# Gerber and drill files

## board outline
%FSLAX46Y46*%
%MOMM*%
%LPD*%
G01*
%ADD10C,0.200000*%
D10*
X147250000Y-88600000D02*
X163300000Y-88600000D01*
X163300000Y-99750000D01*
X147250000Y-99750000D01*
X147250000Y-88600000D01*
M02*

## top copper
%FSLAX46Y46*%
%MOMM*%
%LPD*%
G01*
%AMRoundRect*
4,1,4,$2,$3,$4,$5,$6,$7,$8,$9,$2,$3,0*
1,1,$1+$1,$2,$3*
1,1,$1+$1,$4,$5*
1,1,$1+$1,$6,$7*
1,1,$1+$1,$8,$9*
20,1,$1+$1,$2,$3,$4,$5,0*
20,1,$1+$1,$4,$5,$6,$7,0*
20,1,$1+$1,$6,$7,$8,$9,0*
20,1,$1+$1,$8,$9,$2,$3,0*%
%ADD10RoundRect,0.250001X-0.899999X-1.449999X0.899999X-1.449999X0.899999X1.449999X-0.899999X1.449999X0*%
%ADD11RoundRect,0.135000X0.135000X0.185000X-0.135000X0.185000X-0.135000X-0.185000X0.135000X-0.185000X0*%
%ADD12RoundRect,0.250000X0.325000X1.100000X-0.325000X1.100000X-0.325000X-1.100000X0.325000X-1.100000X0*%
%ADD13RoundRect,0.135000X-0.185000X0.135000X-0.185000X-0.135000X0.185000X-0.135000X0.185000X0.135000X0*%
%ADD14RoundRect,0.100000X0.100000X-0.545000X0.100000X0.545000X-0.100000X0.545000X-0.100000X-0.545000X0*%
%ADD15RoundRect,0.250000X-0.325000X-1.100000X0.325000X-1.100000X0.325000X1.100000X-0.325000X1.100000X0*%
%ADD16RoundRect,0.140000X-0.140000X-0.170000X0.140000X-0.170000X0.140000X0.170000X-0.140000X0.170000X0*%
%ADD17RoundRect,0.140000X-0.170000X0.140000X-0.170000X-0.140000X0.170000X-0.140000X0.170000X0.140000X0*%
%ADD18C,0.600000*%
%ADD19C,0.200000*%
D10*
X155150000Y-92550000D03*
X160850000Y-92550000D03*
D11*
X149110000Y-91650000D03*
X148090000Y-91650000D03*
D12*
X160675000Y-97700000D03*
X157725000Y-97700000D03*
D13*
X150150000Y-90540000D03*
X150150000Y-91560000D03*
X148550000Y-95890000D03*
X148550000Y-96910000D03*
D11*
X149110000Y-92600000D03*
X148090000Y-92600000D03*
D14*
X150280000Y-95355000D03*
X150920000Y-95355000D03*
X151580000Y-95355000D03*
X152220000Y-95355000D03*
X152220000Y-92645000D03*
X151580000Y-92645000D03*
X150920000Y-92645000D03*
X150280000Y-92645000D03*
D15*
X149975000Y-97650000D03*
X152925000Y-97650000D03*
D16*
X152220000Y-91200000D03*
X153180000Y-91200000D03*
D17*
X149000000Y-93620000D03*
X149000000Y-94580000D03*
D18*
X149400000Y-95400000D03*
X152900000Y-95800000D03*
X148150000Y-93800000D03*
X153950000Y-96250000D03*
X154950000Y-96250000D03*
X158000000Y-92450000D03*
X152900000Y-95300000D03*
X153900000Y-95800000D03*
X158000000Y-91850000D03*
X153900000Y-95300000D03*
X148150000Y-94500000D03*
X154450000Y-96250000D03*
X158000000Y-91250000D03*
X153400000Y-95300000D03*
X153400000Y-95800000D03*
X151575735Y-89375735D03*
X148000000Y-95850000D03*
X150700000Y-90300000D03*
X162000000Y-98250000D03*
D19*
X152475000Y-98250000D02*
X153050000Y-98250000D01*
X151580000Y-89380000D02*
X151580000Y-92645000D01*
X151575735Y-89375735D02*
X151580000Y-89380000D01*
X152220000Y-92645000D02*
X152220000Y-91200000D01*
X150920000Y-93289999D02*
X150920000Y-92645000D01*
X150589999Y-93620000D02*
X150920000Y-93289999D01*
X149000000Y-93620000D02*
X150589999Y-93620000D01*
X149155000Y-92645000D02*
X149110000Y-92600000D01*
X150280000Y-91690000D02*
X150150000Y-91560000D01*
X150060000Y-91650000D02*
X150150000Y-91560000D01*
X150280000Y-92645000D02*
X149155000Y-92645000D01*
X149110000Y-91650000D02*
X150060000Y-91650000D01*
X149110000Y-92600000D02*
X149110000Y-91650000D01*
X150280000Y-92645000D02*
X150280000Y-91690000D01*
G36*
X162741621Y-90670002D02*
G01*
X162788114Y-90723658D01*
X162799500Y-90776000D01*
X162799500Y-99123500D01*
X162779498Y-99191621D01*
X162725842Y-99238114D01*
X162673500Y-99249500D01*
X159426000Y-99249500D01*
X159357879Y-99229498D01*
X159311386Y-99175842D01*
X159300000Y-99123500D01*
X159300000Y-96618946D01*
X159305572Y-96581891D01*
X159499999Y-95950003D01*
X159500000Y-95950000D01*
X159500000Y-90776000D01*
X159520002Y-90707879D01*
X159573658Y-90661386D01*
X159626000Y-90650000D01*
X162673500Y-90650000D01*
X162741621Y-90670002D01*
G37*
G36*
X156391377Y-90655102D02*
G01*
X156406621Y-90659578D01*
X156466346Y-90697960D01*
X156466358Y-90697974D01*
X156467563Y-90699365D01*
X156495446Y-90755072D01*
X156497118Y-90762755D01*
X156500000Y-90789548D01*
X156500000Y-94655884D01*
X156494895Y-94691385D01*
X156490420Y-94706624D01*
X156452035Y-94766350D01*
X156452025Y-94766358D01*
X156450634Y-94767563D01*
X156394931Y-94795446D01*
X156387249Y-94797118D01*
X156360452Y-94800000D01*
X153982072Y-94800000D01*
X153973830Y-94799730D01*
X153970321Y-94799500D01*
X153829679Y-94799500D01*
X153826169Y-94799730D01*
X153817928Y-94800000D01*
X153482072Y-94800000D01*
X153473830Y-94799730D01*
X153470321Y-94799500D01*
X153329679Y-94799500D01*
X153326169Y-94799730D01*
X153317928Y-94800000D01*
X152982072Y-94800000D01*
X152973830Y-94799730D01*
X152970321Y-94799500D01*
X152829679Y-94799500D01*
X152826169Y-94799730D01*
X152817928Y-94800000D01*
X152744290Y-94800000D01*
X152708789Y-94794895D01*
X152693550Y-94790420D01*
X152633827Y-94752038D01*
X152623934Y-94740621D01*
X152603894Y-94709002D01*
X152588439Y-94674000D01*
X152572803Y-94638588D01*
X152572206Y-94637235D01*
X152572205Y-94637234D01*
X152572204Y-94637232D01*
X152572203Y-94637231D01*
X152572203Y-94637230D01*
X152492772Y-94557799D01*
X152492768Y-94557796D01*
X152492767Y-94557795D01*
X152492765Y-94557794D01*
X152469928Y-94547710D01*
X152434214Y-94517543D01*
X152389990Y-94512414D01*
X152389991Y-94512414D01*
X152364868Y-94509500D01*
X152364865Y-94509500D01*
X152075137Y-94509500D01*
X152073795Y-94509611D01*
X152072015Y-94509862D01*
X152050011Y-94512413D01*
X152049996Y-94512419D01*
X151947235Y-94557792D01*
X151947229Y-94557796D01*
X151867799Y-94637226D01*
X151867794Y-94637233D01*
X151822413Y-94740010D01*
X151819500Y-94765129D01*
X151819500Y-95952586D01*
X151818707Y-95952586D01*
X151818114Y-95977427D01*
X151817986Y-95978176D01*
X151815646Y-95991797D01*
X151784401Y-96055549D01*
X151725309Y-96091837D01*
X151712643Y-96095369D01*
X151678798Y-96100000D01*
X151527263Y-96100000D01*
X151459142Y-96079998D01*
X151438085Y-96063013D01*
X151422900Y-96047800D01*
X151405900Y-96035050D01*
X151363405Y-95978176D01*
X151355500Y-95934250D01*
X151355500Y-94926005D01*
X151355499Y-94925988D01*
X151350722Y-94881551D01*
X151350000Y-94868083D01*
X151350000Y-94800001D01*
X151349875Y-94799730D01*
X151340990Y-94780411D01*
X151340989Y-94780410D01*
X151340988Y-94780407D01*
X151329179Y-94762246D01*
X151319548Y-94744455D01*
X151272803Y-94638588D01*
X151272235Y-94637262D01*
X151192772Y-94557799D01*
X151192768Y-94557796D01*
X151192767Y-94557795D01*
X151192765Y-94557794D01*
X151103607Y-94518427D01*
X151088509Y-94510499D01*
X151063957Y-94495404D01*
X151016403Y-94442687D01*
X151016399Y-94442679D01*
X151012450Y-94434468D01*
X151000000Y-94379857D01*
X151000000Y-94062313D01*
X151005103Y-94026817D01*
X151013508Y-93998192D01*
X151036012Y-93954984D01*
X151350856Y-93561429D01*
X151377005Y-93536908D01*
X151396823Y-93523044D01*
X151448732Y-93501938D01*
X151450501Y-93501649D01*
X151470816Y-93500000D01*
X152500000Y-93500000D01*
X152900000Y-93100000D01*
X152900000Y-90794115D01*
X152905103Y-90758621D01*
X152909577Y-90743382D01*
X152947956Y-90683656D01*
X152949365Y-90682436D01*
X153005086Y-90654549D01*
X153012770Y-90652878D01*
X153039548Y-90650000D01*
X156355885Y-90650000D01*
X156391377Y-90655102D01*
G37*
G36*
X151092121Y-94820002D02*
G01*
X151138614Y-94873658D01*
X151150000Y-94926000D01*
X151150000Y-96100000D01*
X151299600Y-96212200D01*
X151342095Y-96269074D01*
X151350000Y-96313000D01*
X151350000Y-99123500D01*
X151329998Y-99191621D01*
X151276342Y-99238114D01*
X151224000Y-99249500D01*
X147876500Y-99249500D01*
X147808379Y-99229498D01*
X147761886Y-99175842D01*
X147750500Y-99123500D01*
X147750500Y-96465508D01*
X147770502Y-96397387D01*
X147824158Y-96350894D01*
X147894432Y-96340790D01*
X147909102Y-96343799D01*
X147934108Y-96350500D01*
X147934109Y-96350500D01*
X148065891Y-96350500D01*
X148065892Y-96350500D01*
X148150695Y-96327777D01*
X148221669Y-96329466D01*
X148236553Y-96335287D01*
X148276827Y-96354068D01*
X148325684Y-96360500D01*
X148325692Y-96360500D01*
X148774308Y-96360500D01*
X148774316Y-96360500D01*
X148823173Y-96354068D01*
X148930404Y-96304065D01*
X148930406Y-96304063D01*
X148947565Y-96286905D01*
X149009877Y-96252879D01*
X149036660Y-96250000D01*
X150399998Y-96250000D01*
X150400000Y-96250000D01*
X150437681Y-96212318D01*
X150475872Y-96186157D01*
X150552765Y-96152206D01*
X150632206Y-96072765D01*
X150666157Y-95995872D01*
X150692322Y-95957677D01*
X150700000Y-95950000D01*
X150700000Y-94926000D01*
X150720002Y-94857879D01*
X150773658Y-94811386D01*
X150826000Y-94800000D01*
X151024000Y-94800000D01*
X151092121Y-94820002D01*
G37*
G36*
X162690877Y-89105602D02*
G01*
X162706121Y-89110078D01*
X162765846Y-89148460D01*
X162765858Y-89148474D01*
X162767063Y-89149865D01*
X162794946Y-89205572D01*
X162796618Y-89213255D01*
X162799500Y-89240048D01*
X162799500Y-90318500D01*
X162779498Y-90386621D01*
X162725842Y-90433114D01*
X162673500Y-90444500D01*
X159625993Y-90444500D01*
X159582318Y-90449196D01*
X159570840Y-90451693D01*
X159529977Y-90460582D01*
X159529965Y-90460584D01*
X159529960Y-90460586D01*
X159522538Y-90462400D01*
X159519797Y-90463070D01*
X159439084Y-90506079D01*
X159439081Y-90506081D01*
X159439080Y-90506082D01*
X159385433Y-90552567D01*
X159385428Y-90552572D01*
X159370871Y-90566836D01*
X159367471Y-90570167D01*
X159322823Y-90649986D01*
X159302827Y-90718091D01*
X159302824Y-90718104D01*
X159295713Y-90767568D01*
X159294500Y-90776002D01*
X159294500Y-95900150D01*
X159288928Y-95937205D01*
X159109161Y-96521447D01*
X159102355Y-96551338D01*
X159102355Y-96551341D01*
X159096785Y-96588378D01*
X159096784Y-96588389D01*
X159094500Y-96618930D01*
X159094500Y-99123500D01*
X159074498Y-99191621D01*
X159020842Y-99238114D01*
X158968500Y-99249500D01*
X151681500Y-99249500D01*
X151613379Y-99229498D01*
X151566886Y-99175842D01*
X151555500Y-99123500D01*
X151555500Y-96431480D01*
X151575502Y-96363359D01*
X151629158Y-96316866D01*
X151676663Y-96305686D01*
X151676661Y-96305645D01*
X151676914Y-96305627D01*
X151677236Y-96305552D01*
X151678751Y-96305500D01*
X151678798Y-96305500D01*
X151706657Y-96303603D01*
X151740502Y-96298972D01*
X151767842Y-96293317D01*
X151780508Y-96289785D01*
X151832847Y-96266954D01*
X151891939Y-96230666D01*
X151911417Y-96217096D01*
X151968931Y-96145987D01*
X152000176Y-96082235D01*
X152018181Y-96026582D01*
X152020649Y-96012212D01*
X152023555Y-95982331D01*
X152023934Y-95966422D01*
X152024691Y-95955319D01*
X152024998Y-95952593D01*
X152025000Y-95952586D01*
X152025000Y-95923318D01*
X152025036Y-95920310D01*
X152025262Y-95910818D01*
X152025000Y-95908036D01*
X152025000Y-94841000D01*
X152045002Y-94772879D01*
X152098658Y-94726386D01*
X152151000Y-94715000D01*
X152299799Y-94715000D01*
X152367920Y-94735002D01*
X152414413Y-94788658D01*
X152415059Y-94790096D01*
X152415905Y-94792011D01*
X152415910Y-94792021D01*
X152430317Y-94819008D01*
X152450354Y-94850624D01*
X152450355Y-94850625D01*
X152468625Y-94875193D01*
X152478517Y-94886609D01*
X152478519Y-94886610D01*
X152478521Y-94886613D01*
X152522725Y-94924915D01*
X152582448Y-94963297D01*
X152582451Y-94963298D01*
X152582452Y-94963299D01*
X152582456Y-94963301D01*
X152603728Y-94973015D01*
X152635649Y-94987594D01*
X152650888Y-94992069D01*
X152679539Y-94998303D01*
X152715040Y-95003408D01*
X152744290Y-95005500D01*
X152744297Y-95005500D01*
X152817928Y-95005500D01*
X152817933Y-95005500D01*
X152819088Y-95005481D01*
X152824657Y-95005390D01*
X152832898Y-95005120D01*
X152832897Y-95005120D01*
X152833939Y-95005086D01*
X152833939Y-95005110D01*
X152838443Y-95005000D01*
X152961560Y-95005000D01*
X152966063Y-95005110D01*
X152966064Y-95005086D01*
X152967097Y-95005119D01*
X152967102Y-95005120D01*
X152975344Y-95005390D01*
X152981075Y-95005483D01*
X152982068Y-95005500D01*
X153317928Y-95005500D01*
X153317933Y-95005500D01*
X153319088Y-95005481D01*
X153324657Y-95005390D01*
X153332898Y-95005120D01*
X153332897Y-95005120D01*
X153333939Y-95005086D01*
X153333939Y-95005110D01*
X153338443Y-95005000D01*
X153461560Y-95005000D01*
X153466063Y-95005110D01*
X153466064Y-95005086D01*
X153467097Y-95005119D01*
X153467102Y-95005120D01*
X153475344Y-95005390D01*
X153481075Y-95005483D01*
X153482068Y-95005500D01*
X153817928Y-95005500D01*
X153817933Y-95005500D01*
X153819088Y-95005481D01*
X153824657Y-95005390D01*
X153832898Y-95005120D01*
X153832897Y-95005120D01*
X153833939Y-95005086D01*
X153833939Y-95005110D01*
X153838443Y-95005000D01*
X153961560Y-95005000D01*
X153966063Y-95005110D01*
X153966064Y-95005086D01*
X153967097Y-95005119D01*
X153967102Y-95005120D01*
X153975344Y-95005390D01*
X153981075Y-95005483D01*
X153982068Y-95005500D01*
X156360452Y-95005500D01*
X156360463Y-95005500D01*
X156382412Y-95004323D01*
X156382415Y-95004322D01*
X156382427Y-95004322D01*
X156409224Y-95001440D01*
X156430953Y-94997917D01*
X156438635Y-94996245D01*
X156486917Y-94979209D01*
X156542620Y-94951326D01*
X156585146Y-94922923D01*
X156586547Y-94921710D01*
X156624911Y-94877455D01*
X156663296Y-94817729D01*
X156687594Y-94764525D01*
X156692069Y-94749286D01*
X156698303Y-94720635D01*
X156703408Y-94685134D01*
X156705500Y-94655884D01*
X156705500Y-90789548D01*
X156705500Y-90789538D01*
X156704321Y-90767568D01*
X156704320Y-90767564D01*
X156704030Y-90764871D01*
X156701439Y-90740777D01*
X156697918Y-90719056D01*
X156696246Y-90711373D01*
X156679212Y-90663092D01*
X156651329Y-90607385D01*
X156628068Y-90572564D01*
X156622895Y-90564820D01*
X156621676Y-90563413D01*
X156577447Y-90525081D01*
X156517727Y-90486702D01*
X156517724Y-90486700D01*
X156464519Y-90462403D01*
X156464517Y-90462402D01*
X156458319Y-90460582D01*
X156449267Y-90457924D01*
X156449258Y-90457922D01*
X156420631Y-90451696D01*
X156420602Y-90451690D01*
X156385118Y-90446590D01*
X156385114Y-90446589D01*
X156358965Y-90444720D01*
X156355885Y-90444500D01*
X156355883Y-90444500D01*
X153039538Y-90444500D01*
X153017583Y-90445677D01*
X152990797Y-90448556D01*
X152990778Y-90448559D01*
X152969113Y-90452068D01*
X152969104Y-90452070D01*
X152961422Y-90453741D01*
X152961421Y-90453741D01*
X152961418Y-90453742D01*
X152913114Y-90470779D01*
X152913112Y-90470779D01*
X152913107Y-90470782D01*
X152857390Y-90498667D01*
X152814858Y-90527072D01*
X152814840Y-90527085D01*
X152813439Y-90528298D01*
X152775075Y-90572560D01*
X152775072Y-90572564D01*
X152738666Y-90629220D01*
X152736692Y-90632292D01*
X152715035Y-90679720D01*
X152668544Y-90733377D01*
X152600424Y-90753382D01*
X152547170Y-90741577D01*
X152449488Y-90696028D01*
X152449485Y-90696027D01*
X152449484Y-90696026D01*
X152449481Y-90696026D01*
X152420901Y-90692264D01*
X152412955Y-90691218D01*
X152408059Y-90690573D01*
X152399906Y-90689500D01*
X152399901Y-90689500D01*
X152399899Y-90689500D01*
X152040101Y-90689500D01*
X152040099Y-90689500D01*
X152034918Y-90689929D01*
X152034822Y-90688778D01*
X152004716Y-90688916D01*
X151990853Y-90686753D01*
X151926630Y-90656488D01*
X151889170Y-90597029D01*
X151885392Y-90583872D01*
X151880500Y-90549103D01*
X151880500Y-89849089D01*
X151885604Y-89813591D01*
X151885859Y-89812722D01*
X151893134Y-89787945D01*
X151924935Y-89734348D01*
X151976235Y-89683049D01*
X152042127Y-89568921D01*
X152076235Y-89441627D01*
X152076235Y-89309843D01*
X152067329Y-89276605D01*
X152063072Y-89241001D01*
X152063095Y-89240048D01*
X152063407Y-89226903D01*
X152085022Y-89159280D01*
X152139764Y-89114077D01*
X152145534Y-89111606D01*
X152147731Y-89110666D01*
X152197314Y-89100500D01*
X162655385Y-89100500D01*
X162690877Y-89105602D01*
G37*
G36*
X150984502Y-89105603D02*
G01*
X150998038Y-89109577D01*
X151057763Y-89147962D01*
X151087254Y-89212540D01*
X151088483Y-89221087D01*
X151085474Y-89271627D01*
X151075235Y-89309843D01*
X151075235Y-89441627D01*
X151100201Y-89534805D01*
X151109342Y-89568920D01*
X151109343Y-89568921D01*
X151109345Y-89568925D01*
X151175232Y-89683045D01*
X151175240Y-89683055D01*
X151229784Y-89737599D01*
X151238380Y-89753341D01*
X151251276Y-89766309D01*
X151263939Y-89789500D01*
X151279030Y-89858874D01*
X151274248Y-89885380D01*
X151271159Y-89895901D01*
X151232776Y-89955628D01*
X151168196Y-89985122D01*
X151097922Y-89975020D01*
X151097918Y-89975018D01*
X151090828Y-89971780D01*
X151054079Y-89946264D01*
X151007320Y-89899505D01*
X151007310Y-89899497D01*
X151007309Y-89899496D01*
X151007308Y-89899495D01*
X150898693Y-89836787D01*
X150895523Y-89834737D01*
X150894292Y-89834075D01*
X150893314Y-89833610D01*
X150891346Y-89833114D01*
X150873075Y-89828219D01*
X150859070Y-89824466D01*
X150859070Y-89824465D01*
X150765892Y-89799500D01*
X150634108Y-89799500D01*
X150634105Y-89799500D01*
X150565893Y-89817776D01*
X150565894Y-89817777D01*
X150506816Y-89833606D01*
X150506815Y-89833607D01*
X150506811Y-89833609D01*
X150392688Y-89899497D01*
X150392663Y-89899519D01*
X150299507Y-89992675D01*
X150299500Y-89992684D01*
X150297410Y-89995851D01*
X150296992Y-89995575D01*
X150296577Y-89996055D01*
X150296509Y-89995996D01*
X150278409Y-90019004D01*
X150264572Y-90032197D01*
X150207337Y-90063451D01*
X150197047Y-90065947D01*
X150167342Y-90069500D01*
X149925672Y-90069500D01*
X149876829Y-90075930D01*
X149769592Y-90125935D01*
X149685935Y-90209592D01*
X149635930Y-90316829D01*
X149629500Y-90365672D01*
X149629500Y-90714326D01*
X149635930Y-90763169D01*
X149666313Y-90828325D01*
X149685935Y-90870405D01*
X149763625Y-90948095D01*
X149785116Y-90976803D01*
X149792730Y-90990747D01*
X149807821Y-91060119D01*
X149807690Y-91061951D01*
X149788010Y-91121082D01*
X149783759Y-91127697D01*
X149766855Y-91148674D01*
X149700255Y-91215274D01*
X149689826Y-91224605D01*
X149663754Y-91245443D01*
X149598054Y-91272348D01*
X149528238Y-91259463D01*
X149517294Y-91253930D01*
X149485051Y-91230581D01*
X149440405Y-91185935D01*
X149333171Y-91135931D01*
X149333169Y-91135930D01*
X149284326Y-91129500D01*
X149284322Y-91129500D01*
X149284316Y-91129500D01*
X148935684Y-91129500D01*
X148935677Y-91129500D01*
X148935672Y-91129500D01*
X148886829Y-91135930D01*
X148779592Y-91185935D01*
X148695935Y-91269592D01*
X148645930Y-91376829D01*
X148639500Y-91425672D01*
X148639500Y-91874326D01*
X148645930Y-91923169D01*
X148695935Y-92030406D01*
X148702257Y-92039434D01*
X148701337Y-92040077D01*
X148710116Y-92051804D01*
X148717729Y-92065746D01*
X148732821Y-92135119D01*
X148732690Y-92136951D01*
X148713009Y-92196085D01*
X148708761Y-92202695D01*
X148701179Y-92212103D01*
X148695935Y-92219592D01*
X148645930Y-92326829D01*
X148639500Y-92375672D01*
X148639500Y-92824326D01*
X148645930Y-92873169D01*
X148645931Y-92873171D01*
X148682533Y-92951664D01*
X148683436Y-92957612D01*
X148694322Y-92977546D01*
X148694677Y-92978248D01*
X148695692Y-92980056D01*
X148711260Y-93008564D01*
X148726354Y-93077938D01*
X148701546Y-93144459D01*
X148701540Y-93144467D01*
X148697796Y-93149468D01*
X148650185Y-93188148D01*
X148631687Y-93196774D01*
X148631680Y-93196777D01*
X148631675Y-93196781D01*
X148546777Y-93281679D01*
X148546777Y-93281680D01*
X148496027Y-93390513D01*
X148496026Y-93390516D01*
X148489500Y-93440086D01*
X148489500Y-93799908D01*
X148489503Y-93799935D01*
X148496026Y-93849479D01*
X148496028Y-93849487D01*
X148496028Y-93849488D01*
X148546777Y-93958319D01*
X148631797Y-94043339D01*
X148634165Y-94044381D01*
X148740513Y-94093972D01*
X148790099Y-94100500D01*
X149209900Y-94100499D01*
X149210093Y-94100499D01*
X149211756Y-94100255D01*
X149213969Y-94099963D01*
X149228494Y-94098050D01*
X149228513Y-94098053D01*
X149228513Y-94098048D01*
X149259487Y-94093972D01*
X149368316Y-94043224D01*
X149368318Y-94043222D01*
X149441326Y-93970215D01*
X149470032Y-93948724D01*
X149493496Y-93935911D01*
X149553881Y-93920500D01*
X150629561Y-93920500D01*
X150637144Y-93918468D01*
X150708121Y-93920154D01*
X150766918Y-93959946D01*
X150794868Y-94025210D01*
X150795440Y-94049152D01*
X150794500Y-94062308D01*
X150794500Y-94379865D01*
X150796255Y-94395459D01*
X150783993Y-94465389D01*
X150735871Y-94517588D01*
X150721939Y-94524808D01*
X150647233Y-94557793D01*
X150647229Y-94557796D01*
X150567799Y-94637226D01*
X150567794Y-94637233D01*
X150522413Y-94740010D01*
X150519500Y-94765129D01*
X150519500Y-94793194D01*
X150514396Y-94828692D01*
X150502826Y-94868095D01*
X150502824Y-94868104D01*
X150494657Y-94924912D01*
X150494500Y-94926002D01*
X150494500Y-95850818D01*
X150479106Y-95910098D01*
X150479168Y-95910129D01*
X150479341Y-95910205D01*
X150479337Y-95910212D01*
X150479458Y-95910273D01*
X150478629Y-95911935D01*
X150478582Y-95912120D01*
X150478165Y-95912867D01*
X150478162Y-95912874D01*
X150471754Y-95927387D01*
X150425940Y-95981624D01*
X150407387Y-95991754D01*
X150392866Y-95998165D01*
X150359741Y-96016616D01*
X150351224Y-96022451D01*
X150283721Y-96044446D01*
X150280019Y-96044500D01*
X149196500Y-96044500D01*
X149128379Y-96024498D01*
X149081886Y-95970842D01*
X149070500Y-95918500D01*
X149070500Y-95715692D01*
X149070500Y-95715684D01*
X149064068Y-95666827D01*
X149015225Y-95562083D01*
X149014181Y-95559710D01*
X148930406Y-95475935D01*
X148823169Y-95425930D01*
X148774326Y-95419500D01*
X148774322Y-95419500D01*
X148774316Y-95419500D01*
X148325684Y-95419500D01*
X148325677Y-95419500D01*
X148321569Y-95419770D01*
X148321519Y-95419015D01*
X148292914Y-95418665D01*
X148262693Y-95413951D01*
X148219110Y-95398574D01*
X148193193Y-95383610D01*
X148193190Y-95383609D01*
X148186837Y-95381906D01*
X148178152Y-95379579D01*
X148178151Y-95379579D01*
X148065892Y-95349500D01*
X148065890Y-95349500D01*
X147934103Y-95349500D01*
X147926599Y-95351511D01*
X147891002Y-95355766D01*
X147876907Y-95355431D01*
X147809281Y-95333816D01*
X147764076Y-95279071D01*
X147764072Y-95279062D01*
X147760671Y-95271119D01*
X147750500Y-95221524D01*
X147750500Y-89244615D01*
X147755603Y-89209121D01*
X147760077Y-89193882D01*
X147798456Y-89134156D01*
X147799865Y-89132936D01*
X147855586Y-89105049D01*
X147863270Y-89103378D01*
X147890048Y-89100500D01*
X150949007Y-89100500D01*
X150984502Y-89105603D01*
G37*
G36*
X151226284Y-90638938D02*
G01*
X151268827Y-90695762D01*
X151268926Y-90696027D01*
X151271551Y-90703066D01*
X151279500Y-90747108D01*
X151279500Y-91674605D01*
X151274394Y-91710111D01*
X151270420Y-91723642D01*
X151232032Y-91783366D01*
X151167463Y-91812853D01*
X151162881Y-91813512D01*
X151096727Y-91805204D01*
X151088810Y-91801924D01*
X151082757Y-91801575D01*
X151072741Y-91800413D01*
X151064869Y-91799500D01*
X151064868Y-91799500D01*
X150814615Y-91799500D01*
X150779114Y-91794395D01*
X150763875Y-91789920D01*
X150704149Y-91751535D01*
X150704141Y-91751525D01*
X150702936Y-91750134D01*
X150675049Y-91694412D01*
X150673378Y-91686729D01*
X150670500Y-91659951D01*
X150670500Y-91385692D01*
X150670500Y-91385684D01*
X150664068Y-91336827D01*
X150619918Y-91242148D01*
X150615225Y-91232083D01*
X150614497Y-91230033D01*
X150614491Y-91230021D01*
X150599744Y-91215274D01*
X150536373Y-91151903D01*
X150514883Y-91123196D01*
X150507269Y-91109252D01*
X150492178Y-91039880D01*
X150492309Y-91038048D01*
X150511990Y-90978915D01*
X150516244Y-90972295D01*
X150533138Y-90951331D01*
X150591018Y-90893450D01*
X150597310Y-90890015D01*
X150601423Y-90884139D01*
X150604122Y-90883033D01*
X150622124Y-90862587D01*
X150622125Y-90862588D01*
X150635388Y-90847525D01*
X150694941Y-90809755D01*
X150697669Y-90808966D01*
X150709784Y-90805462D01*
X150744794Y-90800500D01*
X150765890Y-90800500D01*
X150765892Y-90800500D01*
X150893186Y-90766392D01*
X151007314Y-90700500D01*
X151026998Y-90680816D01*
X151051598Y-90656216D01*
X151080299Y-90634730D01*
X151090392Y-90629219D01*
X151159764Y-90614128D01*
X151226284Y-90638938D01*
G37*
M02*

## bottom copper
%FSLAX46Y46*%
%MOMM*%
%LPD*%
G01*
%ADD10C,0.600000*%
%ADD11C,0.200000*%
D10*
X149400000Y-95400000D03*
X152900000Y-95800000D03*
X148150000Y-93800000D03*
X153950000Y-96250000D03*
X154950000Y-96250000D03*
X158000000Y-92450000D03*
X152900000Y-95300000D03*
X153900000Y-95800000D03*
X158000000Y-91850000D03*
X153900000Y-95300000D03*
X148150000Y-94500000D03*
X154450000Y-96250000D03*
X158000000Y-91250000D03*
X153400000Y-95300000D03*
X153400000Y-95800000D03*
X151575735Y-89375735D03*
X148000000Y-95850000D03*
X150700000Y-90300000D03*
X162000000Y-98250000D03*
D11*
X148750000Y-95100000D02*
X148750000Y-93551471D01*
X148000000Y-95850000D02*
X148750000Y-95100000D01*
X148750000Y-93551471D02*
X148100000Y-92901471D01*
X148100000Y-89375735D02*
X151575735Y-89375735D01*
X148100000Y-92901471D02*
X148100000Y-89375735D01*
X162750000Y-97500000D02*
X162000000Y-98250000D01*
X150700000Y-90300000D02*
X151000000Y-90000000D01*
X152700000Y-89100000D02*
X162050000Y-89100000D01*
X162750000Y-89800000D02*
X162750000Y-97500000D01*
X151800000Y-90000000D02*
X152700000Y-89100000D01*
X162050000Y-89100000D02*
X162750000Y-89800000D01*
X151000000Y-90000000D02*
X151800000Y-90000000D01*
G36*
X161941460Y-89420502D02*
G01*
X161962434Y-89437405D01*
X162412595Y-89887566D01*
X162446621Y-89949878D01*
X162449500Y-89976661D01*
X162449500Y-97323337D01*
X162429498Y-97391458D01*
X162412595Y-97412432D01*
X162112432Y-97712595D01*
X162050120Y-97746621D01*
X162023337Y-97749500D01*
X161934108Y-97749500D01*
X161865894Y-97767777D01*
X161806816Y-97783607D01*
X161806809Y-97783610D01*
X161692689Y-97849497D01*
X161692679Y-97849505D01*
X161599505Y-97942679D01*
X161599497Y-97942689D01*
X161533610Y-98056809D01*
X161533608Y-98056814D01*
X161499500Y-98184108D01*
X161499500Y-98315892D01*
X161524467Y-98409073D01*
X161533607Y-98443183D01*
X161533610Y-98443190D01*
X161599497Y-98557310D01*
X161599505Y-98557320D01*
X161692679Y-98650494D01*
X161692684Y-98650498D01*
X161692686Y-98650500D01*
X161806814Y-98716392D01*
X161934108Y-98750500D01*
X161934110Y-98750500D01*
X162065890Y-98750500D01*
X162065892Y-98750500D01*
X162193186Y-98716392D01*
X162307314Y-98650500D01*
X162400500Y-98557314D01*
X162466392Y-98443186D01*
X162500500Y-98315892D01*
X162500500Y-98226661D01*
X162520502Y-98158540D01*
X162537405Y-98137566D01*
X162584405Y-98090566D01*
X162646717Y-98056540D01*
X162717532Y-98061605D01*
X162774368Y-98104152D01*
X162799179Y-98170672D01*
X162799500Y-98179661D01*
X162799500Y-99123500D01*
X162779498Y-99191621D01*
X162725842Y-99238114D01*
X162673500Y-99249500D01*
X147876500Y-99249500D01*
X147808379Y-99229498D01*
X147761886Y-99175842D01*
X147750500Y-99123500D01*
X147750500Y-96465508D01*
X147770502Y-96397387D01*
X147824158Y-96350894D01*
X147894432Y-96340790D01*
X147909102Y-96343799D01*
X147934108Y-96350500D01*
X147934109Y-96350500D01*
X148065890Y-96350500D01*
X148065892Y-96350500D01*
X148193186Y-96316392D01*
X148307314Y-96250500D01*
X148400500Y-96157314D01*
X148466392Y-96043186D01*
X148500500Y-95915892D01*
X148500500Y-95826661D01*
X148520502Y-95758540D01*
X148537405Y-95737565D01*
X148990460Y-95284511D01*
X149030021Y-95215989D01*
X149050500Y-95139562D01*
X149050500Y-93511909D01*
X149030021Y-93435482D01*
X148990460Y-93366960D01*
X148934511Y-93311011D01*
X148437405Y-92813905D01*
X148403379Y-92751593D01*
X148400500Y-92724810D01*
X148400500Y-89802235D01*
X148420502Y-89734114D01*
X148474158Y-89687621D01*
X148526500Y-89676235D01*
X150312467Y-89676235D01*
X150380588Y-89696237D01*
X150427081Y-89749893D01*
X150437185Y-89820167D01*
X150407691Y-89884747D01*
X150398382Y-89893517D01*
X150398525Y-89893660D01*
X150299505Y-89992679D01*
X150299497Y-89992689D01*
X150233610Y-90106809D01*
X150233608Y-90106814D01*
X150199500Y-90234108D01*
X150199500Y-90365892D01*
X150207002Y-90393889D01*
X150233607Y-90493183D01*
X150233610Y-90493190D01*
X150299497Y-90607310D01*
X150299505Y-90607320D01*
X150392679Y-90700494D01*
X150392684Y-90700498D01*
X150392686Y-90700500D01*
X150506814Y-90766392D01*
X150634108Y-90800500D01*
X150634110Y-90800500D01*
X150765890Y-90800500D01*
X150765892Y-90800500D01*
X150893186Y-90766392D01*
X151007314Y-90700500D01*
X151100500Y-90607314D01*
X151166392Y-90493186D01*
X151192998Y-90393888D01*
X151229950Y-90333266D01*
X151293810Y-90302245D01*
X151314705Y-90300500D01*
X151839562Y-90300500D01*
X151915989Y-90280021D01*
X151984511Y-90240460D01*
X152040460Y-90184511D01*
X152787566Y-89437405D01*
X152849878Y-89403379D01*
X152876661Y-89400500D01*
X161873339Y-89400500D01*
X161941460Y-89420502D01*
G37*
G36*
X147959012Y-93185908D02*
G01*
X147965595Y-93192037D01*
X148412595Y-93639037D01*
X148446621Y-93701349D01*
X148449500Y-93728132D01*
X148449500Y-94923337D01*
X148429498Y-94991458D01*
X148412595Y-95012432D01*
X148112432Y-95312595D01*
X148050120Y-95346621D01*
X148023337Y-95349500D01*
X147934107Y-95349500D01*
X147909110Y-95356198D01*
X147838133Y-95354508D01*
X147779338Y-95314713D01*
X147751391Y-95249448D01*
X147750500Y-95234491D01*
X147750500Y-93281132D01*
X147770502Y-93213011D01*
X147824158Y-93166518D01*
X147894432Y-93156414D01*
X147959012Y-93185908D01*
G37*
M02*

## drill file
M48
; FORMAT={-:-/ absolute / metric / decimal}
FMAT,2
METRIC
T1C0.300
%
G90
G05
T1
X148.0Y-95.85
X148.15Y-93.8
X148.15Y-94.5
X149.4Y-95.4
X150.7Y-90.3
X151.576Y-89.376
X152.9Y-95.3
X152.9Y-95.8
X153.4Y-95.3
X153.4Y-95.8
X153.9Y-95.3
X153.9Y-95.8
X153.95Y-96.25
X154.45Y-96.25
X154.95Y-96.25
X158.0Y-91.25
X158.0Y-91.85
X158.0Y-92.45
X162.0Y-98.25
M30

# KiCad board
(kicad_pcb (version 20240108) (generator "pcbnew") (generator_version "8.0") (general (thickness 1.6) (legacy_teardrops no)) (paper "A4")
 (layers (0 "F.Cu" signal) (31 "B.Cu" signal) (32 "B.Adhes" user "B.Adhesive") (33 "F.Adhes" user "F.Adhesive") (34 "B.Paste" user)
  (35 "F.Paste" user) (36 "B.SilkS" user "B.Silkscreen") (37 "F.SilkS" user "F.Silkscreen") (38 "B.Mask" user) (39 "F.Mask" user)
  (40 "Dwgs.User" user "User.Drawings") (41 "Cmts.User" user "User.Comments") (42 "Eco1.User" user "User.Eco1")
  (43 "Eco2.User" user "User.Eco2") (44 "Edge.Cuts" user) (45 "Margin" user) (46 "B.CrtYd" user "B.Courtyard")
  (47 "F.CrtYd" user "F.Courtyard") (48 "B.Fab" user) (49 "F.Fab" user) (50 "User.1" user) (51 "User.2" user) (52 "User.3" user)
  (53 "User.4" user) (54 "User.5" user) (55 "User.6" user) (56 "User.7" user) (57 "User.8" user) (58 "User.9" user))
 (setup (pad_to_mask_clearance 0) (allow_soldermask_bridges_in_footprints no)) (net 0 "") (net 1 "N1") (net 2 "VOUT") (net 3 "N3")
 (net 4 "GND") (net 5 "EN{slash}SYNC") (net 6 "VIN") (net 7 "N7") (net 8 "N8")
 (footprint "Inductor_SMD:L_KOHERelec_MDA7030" (layer "F.Cu") (at 158 92.55)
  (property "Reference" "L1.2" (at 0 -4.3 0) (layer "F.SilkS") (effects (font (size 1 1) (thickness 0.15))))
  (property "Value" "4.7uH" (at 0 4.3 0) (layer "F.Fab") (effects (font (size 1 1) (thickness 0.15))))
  (pad "1" smd roundrect (at -2.85 0) (size 2.3 3.4) (layers "F.Cu" "F.Paste" "F.Mask") (roundrect_rratio 0.108696) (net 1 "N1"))
  (pad "2" smd roundrect (at 2.85 0) (size 2.3 3.4) (layers "F.Cu" "F.Paste" "F.Mask") (roundrect_rratio 0.108696) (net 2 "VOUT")))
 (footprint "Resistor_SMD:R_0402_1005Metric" (layer "F.Cu") (at 148.6 91.65 180)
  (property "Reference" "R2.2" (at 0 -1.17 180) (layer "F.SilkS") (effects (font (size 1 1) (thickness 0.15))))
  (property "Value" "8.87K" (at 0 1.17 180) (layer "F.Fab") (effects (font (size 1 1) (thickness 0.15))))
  (pad "1" smd roundrect (at -0.51 0 180) (size 0.54 0.64) (layers "F.Cu" "F.Paste" "F.Mask") (roundrect_rratio 0.25) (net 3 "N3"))
  (pad "2" smd roundrect (at 0.51 0 180) (size 0.54 0.64) (layers "F.Cu" "F.Paste" "F.Mask") (roundrect_rratio 0.25) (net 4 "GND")))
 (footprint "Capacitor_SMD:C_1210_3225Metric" (layer "F.Cu") (at 159.2 97.7 180)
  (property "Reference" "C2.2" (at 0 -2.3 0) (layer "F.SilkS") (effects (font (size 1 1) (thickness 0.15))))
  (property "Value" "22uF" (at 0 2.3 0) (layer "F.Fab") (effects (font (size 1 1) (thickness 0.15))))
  (pad "1" smd roundrect (at -1.475 0 180) (size 1.15 2.7) (layers "F.Cu" "F.Paste" "F.Mask") (roundrect_rratio 0.217391) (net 2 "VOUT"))
  (pad "2" smd roundrect (at 1.475 0 180) (size 1.15 2.7) (layers "F.Cu" "F.Paste" "F.Mask") (roundrect_rratio 0.217391) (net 4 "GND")))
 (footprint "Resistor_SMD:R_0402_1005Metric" (layer "F.Cu") (at 150.15 91.05 -90)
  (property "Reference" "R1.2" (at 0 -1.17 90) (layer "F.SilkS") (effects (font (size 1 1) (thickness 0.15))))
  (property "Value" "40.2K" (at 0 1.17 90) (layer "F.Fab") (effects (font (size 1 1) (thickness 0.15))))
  (pad "1" smd roundrect (at -0.51 0 270) (size 0.54 0.64) (layers "F.Cu" "F.Paste" "F.Mask") (roundrect_rratio 0.25) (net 2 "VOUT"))
  (pad "2" smd roundrect (at 0.51 0 270) (size 0.54 0.64) (layers "F.Cu" "F.Paste" "F.Mask") (roundrect_rratio 0.25) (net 3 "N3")))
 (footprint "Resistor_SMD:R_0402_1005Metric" (layer "F.Cu") (at 148.55 96.4 -90)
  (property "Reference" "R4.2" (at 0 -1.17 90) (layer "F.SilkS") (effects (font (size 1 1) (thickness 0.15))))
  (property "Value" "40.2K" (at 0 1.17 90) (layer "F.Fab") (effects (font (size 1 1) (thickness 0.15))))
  (pad "1" smd roundrect (at -0.51 0 270) (size 0.54 0.64) (layers "F.Cu" "F.Paste" "F.Mask") (roundrect_rratio 0.25)
   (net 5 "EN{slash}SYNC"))
  (pad "2" smd roundrect (at 0.51 0 270) (size 0.54 0.64) (layers "F.Cu" "F.Paste" "F.Mask") (roundrect_rratio 0.25) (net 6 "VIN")))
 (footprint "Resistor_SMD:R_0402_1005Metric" (layer "F.Cu") (at 148.6 92.6 180)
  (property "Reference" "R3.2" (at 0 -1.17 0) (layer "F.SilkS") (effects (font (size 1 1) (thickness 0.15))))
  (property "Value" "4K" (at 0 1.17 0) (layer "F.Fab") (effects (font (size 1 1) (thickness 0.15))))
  (pad "1" smd roundrect (at -0.51 0 180) (size 0.54 0.64) (layers "F.Cu" "F.Paste" "F.Mask") (roundrect_rratio 0.25) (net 3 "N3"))
  (pad "2" smd roundrect (at 0.51 0 180) (size 0.54 0.64) (layers "F.Cu" "F.Paste" "F.Mask") (roundrect_rratio 0.25) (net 4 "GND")))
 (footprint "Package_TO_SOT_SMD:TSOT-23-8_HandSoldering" (layer "F.Cu") (at 151.25 94 90)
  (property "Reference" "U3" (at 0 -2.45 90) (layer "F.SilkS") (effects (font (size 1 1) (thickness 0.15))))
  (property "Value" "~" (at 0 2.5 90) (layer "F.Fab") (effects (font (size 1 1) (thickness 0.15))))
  (pad "1" smd roundrect (at -1.355 -0.97 90) (size 1.29 0.4) (layers "F.Cu" "F.Paste" "F.Mask") (roundrect_rratio 0.25) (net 4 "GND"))
  (pad "2" smd roundrect (at -1.355 -0.33 90) (size 1.29 0.4) (layers "F.Cu" "F.Paste" "F.Mask") (roundrect_rratio 0.25) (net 6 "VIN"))
  (pad "3" smd roundrect (at -1.355 0.33 90) (size 1.29 0.4) (layers "F.Cu" "F.Paste" "F.Mask") (roundrect_rratio 0.25) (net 1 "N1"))
  (pad "4" smd roundrect (at -1.355 0.97 90) (size 1.29 0.4) (layers "F.Cu" "F.Paste" "F.Mask") (roundrect_rratio 0.25) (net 4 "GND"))
  (pad "5" smd roundrect (at 1.355 0.97 90) (size 1.29 0.4) (layers "F.Cu" "F.Paste" "F.Mask") (roundrect_rratio 0.25) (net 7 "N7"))
  (pad "6" smd roundrect (at 1.355 0.33 90) (size 1.29 0.4) (layers "F.Cu" "F.Paste" "F.Mask") (roundrect_rratio 0.25)
   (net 5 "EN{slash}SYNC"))
  (pad "7" smd roundrect (at 1.355 -0.33 90) (size 1.29 0.4) (layers "F.Cu" "F.Paste" "F.Mask") (roundrect_rratio 0.25) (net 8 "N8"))
  (pad "8" smd roundrect (at 1.355 -0.97 90) (size 1.29 0.4) (layers "F.Cu" "F.Paste" "F.Mask") (roundrect_rratio 0.25) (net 3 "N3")))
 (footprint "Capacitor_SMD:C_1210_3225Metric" (layer "F.Cu") (at 151.45 97.65)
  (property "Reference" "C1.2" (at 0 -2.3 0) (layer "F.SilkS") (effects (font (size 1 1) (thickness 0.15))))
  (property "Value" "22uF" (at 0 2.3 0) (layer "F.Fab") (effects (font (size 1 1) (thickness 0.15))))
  (pad "1" smd roundrect (at -1.475 0) (size 1.15 2.7) (layers "F.Cu" "F.Paste" "F.Mask") (roundrect_rratio 0.217391) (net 6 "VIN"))
  (pad "2" smd roundrect (at 1.475 0) (size 1.15 2.7) (layers "F.Cu" "F.Paste" "F.Mask") (roundrect_rratio 0.217391) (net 4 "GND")))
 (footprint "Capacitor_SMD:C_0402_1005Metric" (layer "F.Cu") (at 152.7 91.2)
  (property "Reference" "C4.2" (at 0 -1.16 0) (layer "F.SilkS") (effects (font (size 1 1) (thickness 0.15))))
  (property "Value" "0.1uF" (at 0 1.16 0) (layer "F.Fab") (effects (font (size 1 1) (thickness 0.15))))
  (pad "1" smd roundrect (at -0.48 0) (size 0.56 0.62) (layers "F.Cu" "F.Paste" "F.Mask") (roundrect_rratio 0.25) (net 7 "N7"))
  (pad "2" smd roundrect (at 0.48 0) (size 0.56 0.62) (layers "F.Cu" "F.Paste" "F.Mask") (roundrect_rratio 0.25) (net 1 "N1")))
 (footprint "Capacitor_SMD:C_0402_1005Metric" (layer "F.Cu") (at 149 94.1 -90)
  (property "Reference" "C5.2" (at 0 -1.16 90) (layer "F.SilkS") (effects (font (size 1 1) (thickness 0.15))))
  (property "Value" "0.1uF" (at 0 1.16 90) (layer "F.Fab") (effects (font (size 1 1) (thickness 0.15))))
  (pad "1" smd roundrect (at -0.48 0 270) (size 0.56 0.62) (layers "F.Cu" "F.Paste" "F.Mask") (roundrect_rratio 0.25) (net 8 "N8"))
  (pad "2" smd roundrect (at 0.48 0 270) (size 0.56 0.62) (layers "F.Cu" "F.Paste" "F.Mask") (roundrect_rratio 0.25) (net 4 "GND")))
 (gr_rect (start 147.25 88.6) (end 163.3 99.75) (stroke (width 0.2) (type default)) (fill none) (layer "Edge.Cuts"))
 (segment (start 152.475 98.25) (end 153.05 98.25) (width 0.2) (layer "F.Cu") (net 4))
 (via (at 149.4 95.4) (size 0.6) (drill 0.3) (layers "F.Cu" "B.Cu") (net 4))
 (via (at 152.9 95.8) (size 0.6) (drill 0.3) (layers "F.Cu" "B.Cu") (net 4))
 (via (at 148.15 93.8) (size 0.6) (drill 0.3) (layers "F.Cu" "B.Cu") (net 4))
 (via (at 153.95 96.25) (size 0.6) (drill 0.3) (layers "F.Cu" "B.Cu") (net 4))
 (via (at 154.95 96.25) (size 0.6) (drill 0.3) (layers "F.Cu" "B.Cu") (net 4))
 (via (at 158 92.45) (size 0.6) (drill 0.3) (layers "F.Cu" "B.Cu") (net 4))
 (via (at 152.9 95.3) (size 0.6) (drill 0.3) (layers "F.Cu" "B.Cu") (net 4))
 (via (at 153.9 95.8) (size 0.6) (drill 0.3) (layers "F.Cu" "B.Cu") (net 4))
 (via (at 158 91.85) (size 0.6) (drill 0.3) (layers "F.Cu" "B.Cu") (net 4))
 (via (at 153.9 95.3) (size 0.6) (drill 0.3) (layers "F.Cu" "B.Cu") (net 4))
 (via (at 148.15 94.5) (size 0.6) (drill 0.3) (layers "F.Cu" "B.Cu") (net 4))
 (via (at 154.45 96.25) (size 0.6) (drill 0.3) (layers "F.Cu" "B.Cu") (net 4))
 (via (at 158 91.25) (size 0.6) (drill 0.3) (layers "F.Cu" "B.Cu") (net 4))
 (via (at 153.4 95.3) (size 0.6) (drill 0.3) (layers "F.Cu" "B.Cu") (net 4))
 (via (at 153.4 95.8) (size 0.6) (drill 0.3) (layers "F.Cu" "B.Cu") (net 4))
 (segment (start 151.58 89.38) (end 151.58 92.645) (width 0.2) (layer "F.Cu") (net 5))
 (segment (start 151.575735 89.375735) (end 151.58 89.38) (width 0.2) (layer "F.Cu") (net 5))
 (via (at 151.575735 89.375735) (size 0.6) (drill 0.3) (layers "F.Cu" "B.Cu") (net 5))
 (via (at 148 95.85) (size 0.6) (drill 0.3) (layers "F.Cu" "B.Cu") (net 5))
 (segment (start 148.75 95.1) (end 148.75 93.551471) (width 0.2) (layer "B.Cu") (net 5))
 (segment (start 148 95.85) (end 148.75 95.1) (width 0.2) (layer "B.Cu") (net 5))
 (segment (start 148.75 93.551471) (end 148.1 92.901471) (width 0.2) (layer "B.Cu") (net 5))
 (segment (start 148.1 89.375735) (end 151.575735 89.375735) (width 0.2) (layer "B.Cu") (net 5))
 (segment (start 148.1 92.901471) (end 148.1 89.375735) (width 0.2) (layer "B.Cu") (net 5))
 (via (at 150.7 90.3) (size 0.6) (drill 0.3) (layers "F.Cu" "B.Cu") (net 2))
 (via (at 162 98.25) (size 0.6) (drill 0.3) (layers "F.Cu" "B.Cu") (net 2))
 (segment (start 162.75 97.5) (end 162 98.25) (width 0.2) (layer "B.Cu") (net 2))
 (segment (start 150.7 90.3) (end 151 90) (width 0.2) (layer "B.Cu") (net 2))
 (segment (start 152.7 89.1) (end 162.05 89.1) (width 0.2) (layer "B.Cu") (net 2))
 (segment (start 162.75 89.8) (end 162.75 97.5) (width 0.2) (layer "B.Cu") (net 2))
 (segment (start 151.8 90) (end 152.7 89.1) (width 0.2) (layer "B.Cu") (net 2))
 (segment (start 162.05 89.1) (end 162.75 89.8) (width 0.2) (layer "B.Cu") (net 2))
 (segment (start 151 90) (end 151.8 90) (width 0.2) (layer "B.Cu") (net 2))
 (segment (start 152.22 92.645) (end 152.22 91.2) (width 0.2) (layer "F.Cu") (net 7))
 (segment (start 150.92 93.289999) (end 150.92 92.645) (width 0.2) (layer "F.Cu") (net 8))
 (segment (start 150.589999 93.62) (end 150.92 93.289999) (width 0.2) (layer "F.Cu") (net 8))
 (segment (start 149 93.62) (end 150.589999 93.62) (width 0.2) (layer "F.Cu") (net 8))
 (segment (start 149.155 92.645) (end 149.11 92.6) (width 0.2) (layer "F.Cu") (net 3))
 (segment (start 150.28 91.69) (end 150.15 91.56) (width 0.2) (layer "F.Cu") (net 3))
 (segment (start 150.06 91.65) (end 150.15 91.56) (width 0.2) (layer "F.Cu") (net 3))
 (segment (start 150.28 92.645) (end 149.155 92.645) (width 0.2) (layer "F.Cu") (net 3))
 (segment (start 149.11 91.65) (end 150.06 91.65) (width 0.2) (layer "F.Cu") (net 3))
 (segment (start 149.11 92.6) (end 149.11 91.65) (width 0.2) (layer "F.Cu") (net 3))
 (segment (start 150.28 92.645) (end 150.28 91.69) (width 0.2) (layer "F.Cu") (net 3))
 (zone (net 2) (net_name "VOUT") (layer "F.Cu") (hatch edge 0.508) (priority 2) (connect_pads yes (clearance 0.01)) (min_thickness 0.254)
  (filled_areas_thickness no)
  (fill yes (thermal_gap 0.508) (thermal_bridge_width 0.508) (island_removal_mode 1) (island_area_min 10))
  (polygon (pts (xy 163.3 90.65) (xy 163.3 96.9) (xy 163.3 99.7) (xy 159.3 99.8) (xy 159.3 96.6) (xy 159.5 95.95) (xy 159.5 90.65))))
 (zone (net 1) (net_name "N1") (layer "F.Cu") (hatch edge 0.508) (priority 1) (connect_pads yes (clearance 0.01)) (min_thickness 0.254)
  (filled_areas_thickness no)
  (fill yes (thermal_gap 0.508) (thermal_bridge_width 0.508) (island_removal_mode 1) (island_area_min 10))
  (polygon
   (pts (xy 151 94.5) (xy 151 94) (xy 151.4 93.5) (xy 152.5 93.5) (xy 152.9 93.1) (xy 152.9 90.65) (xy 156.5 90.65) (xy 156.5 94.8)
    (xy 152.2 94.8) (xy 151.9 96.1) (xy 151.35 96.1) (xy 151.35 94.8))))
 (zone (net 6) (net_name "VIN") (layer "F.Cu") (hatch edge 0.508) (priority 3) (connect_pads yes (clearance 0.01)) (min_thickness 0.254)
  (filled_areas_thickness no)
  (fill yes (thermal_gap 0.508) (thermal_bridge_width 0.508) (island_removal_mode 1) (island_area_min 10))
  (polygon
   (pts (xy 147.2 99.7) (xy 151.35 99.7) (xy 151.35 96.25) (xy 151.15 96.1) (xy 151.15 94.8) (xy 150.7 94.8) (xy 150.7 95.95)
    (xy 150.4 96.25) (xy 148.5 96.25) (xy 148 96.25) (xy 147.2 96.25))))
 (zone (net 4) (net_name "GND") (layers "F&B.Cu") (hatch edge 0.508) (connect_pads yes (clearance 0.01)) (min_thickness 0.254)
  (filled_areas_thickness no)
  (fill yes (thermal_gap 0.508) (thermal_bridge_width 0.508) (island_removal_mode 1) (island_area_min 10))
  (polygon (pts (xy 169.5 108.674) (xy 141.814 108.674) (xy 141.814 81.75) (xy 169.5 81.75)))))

